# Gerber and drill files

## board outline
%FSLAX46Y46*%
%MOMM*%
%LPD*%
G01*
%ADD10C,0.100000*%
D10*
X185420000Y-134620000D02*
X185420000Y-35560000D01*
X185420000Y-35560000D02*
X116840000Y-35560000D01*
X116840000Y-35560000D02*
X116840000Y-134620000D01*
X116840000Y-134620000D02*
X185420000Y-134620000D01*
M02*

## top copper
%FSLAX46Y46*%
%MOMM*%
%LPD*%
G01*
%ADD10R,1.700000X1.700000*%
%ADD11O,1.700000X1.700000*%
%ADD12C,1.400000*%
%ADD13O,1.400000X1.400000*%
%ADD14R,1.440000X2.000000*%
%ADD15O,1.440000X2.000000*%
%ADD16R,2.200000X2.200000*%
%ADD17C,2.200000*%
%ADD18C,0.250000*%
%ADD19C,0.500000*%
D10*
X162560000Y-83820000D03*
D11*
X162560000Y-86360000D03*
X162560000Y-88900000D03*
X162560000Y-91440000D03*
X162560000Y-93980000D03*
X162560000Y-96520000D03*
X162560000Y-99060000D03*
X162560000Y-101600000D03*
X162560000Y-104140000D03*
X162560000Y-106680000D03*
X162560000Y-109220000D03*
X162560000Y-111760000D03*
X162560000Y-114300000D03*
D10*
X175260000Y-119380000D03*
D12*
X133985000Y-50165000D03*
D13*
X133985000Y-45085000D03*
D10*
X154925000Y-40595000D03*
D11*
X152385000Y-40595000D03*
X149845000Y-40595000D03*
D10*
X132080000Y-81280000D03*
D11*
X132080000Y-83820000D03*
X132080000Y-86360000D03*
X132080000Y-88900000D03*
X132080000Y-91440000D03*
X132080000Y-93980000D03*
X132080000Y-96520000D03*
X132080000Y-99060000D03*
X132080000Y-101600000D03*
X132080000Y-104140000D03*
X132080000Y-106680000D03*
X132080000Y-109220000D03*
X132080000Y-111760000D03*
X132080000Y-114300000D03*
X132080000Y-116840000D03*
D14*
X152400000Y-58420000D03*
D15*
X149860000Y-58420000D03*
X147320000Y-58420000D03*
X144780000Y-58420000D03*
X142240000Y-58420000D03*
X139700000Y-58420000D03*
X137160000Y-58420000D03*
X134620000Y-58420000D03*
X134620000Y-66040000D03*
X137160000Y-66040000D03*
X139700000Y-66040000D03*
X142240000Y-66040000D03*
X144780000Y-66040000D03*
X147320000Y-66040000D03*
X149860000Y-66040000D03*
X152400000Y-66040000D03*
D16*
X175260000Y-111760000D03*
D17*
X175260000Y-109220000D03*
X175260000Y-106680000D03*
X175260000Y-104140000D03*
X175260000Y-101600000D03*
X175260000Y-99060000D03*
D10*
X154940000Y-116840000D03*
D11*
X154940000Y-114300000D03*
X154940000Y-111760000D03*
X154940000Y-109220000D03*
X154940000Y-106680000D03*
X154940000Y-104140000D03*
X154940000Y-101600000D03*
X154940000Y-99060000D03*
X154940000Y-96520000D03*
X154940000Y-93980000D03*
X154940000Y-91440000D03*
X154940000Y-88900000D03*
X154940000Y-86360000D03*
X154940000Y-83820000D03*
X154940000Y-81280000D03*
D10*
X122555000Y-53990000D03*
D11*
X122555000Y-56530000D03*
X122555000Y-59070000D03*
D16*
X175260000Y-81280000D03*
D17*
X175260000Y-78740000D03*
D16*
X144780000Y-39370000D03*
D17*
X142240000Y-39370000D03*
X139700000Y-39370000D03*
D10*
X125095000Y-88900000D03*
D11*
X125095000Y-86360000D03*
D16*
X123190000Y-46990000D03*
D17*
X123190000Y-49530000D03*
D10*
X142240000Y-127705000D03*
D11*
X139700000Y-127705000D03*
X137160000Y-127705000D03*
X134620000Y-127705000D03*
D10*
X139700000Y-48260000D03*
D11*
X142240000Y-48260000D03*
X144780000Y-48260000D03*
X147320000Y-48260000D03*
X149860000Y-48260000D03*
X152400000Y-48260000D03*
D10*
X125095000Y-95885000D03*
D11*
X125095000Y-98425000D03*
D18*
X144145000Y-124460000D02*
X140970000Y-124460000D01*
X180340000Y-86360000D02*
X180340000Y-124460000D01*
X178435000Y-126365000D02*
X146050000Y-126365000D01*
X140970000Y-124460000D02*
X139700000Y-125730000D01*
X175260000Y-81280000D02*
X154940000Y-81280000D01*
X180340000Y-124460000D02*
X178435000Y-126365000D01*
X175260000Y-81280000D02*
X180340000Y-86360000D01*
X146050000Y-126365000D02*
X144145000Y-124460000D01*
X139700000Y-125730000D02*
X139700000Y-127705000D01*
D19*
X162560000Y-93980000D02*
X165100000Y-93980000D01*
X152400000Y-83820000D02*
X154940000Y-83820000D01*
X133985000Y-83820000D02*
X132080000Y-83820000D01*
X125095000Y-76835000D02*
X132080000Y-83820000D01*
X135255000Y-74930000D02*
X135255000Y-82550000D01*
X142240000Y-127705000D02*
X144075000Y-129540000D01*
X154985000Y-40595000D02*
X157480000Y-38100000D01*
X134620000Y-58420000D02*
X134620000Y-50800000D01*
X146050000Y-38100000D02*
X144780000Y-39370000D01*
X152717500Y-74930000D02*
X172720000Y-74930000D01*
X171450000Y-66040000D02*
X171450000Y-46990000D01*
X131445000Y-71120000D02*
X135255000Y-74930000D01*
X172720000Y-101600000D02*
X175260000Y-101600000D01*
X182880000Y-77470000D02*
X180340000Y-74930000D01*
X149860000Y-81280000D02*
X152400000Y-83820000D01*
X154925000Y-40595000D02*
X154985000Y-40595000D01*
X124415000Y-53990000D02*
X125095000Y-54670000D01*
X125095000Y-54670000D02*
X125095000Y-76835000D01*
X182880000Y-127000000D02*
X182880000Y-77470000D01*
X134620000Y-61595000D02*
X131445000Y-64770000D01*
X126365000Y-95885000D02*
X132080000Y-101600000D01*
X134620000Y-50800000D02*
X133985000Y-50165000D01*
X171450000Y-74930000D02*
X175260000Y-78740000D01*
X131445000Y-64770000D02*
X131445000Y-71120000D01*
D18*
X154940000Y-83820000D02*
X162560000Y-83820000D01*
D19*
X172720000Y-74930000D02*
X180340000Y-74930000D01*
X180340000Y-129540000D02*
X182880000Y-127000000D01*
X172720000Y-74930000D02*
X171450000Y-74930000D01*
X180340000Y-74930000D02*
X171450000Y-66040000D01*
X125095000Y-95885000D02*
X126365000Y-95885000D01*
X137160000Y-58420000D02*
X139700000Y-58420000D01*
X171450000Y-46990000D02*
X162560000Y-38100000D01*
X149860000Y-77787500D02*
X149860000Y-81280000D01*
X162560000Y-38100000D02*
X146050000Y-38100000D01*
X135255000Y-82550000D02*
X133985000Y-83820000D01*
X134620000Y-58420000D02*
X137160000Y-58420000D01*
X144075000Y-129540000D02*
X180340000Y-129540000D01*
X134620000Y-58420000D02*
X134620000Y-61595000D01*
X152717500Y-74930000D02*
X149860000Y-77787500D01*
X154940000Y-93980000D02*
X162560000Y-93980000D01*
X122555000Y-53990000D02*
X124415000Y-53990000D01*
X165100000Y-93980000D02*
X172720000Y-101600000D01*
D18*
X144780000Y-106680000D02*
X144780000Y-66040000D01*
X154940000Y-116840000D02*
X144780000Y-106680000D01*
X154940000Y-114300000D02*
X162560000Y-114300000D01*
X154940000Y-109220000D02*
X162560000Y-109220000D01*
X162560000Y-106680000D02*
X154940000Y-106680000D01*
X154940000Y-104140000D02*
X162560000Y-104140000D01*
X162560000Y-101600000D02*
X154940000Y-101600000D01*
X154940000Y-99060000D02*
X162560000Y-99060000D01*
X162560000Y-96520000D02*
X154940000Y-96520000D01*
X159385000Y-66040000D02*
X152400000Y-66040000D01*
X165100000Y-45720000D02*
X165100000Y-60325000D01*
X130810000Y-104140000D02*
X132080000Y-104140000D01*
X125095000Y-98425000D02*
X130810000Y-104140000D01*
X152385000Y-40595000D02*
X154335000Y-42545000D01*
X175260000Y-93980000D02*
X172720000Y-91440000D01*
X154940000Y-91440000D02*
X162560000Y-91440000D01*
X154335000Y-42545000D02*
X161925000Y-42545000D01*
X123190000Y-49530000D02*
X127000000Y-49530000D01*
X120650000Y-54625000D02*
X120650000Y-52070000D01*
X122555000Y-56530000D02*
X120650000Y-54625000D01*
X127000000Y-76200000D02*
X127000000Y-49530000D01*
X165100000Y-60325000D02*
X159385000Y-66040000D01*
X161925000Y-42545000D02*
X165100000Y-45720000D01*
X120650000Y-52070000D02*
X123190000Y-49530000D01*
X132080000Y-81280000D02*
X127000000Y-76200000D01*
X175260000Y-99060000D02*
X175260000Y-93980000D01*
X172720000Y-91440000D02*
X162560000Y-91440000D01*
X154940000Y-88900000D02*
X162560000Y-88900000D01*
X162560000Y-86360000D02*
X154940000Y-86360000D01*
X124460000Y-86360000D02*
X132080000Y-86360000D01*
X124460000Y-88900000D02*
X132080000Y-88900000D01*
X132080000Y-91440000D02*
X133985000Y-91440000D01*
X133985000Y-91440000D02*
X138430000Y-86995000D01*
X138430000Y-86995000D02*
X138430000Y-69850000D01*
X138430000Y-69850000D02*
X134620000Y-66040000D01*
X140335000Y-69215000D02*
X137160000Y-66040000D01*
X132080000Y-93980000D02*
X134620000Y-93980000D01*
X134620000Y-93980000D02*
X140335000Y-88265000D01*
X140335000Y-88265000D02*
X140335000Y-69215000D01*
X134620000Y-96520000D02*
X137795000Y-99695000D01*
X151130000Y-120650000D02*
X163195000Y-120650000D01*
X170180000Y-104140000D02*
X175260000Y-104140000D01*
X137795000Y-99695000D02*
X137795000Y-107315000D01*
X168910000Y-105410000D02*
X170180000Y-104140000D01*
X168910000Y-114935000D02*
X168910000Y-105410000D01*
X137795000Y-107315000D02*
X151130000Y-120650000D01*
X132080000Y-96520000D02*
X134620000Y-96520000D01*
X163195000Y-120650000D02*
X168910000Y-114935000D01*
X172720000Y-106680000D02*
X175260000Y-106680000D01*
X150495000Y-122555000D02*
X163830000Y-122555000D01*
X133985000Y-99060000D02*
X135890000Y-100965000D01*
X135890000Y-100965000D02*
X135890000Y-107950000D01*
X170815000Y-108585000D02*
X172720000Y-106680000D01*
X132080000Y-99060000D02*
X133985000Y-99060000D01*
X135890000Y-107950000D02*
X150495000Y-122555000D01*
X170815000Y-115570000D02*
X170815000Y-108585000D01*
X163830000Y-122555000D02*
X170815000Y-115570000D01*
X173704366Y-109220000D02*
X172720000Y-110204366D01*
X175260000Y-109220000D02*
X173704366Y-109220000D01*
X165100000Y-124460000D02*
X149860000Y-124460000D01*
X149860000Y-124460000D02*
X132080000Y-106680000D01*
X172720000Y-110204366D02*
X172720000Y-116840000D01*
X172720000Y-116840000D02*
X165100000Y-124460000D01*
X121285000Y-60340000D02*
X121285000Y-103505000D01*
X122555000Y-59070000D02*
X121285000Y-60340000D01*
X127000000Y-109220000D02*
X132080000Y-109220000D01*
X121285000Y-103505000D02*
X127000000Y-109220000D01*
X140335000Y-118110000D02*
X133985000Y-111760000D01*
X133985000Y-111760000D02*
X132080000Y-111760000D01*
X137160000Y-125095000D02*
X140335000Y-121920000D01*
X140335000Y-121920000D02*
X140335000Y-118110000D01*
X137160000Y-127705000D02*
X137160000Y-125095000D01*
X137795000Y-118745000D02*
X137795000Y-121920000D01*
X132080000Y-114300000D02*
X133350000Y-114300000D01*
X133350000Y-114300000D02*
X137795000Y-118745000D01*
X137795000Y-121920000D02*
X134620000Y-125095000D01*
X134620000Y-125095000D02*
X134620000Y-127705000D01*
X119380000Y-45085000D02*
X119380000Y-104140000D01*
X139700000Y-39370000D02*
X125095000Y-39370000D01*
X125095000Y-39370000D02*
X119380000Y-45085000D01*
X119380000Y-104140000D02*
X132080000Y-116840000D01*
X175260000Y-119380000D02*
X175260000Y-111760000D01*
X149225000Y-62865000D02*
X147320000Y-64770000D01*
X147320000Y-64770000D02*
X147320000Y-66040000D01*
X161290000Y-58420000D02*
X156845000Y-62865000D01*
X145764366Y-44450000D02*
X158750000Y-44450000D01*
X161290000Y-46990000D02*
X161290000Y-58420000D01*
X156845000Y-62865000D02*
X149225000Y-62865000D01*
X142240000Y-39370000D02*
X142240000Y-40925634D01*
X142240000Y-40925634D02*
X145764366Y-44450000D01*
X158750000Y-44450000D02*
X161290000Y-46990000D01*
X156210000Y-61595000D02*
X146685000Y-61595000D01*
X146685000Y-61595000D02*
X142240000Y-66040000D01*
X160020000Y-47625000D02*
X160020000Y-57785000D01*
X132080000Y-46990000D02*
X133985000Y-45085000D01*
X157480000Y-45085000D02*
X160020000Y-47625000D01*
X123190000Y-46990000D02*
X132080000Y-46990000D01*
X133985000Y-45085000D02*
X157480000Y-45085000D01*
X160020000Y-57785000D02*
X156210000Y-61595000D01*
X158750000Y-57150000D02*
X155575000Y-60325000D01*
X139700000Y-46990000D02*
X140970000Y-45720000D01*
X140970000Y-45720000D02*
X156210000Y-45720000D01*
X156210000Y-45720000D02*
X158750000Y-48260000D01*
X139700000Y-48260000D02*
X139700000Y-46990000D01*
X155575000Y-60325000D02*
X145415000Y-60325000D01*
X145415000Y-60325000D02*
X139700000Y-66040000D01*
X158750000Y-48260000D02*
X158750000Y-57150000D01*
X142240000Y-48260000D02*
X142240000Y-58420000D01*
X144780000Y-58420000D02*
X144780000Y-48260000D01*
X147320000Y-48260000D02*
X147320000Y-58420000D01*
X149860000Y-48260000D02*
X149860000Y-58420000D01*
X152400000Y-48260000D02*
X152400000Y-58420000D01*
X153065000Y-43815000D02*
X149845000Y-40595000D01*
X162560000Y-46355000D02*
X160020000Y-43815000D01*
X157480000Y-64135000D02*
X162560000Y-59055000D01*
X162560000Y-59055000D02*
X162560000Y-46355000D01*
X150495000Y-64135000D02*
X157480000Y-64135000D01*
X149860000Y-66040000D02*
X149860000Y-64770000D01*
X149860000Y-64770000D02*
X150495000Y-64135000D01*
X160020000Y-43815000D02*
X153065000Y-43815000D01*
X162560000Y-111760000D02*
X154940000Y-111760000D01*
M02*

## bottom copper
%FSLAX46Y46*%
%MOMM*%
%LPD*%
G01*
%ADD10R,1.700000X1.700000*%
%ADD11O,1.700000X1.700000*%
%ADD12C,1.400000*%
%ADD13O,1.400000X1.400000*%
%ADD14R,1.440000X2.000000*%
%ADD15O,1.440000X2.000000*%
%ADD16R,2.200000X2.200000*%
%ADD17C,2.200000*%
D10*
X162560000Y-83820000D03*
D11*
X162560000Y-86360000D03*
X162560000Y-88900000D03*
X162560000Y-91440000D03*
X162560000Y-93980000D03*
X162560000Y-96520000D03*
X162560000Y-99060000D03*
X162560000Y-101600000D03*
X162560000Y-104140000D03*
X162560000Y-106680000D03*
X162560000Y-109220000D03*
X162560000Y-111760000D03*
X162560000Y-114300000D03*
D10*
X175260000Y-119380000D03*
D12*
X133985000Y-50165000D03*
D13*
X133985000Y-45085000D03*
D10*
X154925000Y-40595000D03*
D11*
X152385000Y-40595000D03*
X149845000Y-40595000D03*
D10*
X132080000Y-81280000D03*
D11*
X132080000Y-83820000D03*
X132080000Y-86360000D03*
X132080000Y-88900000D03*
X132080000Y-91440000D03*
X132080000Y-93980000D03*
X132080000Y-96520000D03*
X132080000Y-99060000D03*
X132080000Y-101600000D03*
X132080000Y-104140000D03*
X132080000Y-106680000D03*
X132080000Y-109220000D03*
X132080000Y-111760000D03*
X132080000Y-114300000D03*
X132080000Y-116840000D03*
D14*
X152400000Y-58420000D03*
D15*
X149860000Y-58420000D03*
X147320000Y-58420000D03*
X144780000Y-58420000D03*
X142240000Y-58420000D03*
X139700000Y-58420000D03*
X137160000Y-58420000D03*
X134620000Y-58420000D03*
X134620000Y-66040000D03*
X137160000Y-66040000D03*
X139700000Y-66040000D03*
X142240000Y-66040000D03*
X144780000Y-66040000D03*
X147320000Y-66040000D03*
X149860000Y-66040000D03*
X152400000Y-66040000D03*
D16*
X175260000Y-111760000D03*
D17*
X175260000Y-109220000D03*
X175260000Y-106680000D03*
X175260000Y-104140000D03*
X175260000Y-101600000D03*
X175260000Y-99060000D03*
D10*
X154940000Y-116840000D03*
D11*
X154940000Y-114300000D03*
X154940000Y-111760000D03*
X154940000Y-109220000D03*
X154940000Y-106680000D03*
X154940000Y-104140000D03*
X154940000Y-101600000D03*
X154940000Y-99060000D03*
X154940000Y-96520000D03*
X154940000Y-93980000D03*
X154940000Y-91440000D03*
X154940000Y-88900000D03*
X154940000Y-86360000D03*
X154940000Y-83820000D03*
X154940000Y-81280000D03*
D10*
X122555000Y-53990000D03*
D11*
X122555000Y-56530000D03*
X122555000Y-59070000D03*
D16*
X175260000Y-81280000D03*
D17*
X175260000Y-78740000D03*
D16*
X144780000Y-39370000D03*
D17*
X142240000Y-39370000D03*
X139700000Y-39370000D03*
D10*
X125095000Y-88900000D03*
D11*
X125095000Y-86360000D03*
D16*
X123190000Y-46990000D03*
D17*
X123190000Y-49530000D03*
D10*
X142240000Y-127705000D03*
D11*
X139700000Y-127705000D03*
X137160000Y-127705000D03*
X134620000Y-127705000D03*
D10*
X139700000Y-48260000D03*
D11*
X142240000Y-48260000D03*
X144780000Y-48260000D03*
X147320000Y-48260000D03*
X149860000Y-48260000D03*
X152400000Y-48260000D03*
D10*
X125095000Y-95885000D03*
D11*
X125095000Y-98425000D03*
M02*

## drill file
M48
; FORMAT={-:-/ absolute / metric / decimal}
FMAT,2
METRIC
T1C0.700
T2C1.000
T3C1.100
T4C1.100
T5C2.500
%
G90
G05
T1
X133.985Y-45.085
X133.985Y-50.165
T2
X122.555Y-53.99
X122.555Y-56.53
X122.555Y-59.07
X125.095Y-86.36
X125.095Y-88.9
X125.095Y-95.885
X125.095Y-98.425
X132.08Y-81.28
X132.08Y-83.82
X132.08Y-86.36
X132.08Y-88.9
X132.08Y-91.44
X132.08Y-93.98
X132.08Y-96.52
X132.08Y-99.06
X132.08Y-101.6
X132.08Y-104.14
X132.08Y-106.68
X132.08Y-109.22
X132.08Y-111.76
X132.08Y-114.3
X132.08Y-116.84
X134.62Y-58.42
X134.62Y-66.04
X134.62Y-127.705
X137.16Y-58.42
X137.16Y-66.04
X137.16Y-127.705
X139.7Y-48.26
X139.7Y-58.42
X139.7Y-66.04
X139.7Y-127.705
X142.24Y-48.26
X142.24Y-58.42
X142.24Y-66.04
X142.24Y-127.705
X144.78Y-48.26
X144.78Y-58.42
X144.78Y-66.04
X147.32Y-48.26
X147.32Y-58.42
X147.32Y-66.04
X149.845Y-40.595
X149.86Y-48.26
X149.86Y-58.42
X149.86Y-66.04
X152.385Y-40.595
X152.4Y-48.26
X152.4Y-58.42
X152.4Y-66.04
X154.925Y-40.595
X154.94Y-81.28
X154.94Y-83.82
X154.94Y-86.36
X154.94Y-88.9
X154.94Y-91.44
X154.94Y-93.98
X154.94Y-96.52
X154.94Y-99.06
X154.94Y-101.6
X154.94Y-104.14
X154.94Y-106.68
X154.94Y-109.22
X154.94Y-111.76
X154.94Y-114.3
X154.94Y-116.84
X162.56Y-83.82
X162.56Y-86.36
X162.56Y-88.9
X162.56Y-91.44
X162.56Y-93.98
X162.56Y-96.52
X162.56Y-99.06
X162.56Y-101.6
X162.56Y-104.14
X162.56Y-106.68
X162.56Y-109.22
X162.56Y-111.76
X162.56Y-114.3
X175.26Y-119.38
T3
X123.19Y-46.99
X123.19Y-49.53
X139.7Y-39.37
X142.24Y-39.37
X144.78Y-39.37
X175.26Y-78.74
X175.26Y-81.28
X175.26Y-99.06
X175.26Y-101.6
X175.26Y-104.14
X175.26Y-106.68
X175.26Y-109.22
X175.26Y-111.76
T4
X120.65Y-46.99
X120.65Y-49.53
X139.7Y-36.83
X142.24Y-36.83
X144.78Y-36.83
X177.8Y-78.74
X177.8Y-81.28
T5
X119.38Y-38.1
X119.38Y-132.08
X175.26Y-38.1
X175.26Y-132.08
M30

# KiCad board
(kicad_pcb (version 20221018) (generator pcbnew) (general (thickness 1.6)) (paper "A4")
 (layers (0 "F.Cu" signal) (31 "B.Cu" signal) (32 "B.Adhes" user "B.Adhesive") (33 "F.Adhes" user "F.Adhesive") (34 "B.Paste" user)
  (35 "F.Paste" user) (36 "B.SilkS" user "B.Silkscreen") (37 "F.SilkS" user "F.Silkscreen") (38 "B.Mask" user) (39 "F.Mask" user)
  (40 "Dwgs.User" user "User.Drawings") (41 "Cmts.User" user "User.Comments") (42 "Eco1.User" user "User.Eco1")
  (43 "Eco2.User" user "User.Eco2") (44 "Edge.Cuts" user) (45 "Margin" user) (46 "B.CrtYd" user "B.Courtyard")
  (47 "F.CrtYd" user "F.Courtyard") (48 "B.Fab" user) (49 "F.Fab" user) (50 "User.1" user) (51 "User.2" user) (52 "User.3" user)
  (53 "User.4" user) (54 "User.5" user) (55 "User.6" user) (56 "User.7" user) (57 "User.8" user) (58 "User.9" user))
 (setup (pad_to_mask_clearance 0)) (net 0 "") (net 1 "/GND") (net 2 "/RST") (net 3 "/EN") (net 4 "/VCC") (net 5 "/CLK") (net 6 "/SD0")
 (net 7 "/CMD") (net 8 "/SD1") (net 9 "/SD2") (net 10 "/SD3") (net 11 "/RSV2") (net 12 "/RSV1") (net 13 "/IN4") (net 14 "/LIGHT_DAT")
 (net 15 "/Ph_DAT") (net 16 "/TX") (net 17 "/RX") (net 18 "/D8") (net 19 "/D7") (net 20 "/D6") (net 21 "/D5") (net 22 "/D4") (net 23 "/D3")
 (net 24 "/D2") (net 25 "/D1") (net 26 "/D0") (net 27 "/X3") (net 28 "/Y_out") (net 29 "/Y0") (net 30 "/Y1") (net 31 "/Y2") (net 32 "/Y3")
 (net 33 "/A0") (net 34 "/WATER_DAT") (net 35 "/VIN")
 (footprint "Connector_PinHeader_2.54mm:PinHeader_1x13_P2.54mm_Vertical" (layer "F.Cu") (at 162.56 83.82)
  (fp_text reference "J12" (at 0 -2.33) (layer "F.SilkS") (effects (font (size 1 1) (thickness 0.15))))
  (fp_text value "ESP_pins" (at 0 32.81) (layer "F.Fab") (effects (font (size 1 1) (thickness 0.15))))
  (pad "1" thru_hole rect (at 0 0) (size 1.7 1.7) (drill 1) (layers "*.Cu" "*.Mask") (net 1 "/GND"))
  (pad "2" thru_hole oval (at 0 2.54) (size 1.7 1.7) (drill 1) (layers "*.Cu" "*.Mask") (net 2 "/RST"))
  (pad "3" thru_hole oval (at 0 5.08) (size 1.7 1.7) (drill 1) (layers "*.Cu" "*.Mask") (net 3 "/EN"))
  (pad "4" thru_hole oval (at 0 7.62) (size 1.7 1.7) (drill 1) (layers "*.Cu" "*.Mask") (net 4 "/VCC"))
  (pad "5" thru_hole oval (at 0 10.16) (size 1.7 1.7) (drill 1) (layers "*.Cu" "*.Mask") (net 1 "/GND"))
  (pad "6" thru_hole oval (at 0 12.7) (size 1.7 1.7) (drill 1) (layers "*.Cu" "*.Mask") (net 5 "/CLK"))
  (pad "7" thru_hole oval (at 0 15.24) (size 1.7 1.7) (drill 1) (layers "*.Cu" "*.Mask") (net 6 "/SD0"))
  (pad "8" thru_hole oval (at 0 17.78) (size 1.7 1.7) (drill 1) (layers "*.Cu" "*.Mask") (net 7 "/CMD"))
  (pad "9" thru_hole oval (at 0 20.32) (size 1.7 1.7) (drill 1) (layers "*.Cu" "*.Mask") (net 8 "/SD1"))
  (pad "10" thru_hole oval (at 0 22.86) (size 1.7 1.7) (drill 1) (layers "*.Cu" "*.Mask") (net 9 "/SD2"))
  (pad "11" thru_hole oval (at 0 25.4) (size 1.7 1.7) (drill 1) (layers "*.Cu" "*.Mask") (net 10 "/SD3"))
  (pad "12" thru_hole oval (at 0 27.94) (size 1.7 1.7) (drill 1) (layers "*.Cu" "*.Mask") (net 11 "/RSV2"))
  (pad "13" thru_hole oval (at 0 30.48) (size 1.7 1.7) (drill 1) (layers "*.Cu" "*.Mask") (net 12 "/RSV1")))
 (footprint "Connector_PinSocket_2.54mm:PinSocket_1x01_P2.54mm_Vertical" (layer "F.Cu") (at 175.26 119.38)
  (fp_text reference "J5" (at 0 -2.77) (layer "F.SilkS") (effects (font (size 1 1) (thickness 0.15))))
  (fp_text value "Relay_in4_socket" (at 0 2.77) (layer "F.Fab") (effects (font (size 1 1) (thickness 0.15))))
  (pad "1" thru_hole rect (at 0 0) (size 1.7 1.7) (drill 1) (layers "*.Cu" "*.Mask") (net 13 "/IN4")))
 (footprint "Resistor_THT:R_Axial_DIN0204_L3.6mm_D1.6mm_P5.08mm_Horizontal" (layer "F.Cu") (at 133.985 50.165 90)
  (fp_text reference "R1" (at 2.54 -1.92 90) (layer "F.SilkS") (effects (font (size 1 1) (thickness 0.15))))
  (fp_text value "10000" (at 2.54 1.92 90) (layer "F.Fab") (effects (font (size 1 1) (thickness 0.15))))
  (pad "1" thru_hole circle (at 0 0 90) (size 1.4 1.4) (drill 0.7) (layers "*.Cu" "*.Mask") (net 1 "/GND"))
  (pad "2" thru_hole oval (at 5.08 0 90) (size 1.4 1.4) (drill 0.7) (layers "*.Cu" "*.Mask") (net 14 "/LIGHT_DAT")))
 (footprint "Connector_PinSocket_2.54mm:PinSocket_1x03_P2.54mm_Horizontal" (layer "F.Cu") (at 154.925 40.595 -90)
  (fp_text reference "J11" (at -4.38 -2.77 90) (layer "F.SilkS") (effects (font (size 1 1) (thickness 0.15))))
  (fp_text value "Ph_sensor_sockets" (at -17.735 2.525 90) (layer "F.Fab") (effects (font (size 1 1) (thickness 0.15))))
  (pad "1" thru_hole rect (at 0 0 270) (size 1.7 1.7) (drill 1) (layers "*.Cu" "*.Mask") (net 1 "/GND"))
  (pad "2" thru_hole oval (at 0 2.54 270) (size 1.7 1.7) (drill 1) (layers "*.Cu" "*.Mask") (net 4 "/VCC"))
  (pad "3" thru_hole oval (at 0 5.08 270) (size 1.7 1.7) (drill 1) (layers "*.Cu" "*.Mask") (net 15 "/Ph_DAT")))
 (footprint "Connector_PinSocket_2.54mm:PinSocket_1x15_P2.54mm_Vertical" (layer "F.Cu") (at 132.08 81.28)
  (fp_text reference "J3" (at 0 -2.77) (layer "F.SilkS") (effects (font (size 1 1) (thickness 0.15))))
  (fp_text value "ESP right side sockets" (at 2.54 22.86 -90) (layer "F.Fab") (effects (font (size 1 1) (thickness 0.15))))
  (pad "1" thru_hole rect (at 0 0) (size 1.7 1.7) (drill 1) (layers "*.Cu" "*.Mask") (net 4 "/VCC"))
  (pad "2" thru_hole oval (at 0 2.54) (size 1.7 1.7) (drill 1) (layers "*.Cu" "*.Mask") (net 1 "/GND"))
  (pad "3" thru_hole oval (at 0 5.08) (size 1.7 1.7) (drill 1) (layers "*.Cu" "*.Mask") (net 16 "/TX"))
  (pad "4" thru_hole oval (at 0 7.62) (size 1.7 1.7) (drill 1) (layers "*.Cu" "*.Mask") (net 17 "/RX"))
  (pad "5" thru_hole oval (at 0 10.16) (size 1.7 1.7) (drill 1) (layers "*.Cu" "*.Mask") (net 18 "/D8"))
  (pad "6" thru_hole oval (at 0 12.7) (size 1.7 1.7) (drill 1) (layers "*.Cu" "*.Mask") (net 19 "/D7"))
  (pad "7" thru_hole oval (at 0 15.24) (size 1.7 1.7) (drill 1) (layers "*.Cu" "*.Mask") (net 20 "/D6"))
  (pad "8" thru_hole oval (at 0 17.78) (size 1.7 1.7) (drill 1) (layers "*.Cu" "*.Mask") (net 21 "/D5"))
  (pad "9" thru_hole oval (at 0 20.32) (size 1.7 1.7) (drill 1) (layers "*.Cu" "*.Mask") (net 1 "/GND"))
  (pad "10" thru_hole oval (at 0 22.86) (size 1.7 1.7) (drill 1) (layers "*.Cu" "*.Mask") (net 4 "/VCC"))
  (pad "11" thru_hole oval (at 0 25.4) (size 1.7 1.7) (drill 1) (layers "*.Cu" "*.Mask") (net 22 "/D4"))
  (pad "12" thru_hole oval (at 0 27.94) (size 1.7 1.7) (drill 1) (layers "*.Cu" "*.Mask") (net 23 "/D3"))
  (pad "13" thru_hole oval (at 0 30.48) (size 1.7 1.7) (drill 1) (layers "*.Cu" "*.Mask") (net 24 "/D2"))
  (pad "14" thru_hole oval (at 0 33.02) (size 1.7 1.7) (drill 1) (layers "*.Cu" "*.Mask") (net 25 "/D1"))
  (pad "15" thru_hole oval (at 0 35.56) (size 1.7 1.7) (drill 1) (layers "*.Cu" "*.Mask") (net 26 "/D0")))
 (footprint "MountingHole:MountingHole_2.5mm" (layer "F.Cu") (at 119.38 38.1)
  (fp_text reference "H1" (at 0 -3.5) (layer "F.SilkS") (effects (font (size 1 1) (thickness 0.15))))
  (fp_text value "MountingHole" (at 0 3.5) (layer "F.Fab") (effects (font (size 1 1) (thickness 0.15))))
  (pad "" np_thru_hole circle (at 0 0) (size 2.5 2.5) (drill 2.5) (layers "*.Cu" "*.Mask")))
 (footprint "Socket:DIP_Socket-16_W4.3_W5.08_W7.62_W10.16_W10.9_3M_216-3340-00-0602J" (layer "F.Cu") (at 152.4 58.42 -90)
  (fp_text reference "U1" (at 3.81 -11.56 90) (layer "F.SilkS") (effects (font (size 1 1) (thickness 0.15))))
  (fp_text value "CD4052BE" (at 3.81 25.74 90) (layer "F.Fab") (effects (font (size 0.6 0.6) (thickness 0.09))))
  (pad "1" thru_hole rect (at 0 0 270) (size 2 1.44) (drill 1) (layers "*.Cu" "*.Mask") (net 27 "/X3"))
  (pad "2" thru_hole oval (at 0 2.54 270) (size 2 1.44) (drill 1) (layers "*.Cu" "*.Mask") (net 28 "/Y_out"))
  (pad "3" thru_hole oval (at 0 5.08 270) (size 2 1.44) (drill 1) (layers "*.Cu" "*.Mask") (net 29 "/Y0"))
  (pad "4" thru_hole oval (at 0 7.62 270) (size 2 1.44) (drill 1) (layers "*.Cu" "*.Mask") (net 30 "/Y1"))
  (pad "5" thru_hole oval (at 0 10.16 270) (size 2 1.44) (drill 1) (layers "*.Cu" "*.Mask") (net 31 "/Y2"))
  (pad "6" thru_hole oval (at 0 12.7 270) (size 2 1.44) (drill 1) (layers "*.Cu" "*.Mask") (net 1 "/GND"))
  (pad "7" thru_hole oval (at 0 15.24 270) (size 2 1.44) (drill 1) (layers "*.Cu" "*.Mask") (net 1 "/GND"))
  (pad "8" thru_hole oval (at 0 17.78 270) (size 2 1.44) (drill 1) (layers "*.Cu" "*.Mask") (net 1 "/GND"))
  (pad "9" thru_hole oval (at 7.62 17.78 270) (size 2 1.44) (drill 1) (layers "*.Cu" "*.Mask") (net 18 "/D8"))
  (pad "10" thru_hole oval (at 7.62 15.24 270) (size 2 1.44) (drill 1) (layers "*.Cu" "*.Mask") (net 19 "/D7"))
  (pad "11" thru_hole oval (at 7.62 12.7 270) (size 2 1.44) (drill 1) (layers "*.Cu" "*.Mask") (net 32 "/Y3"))
  (pad "12" thru_hole oval (at 7.62 10.16 270) (size 2 1.44) (drill 1) (layers "*.Cu" "*.Mask") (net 14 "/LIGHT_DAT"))
  (pad "13" thru_hole oval (at 7.62 7.62 270) (size 2 1.44) (drill 1) (layers "*.Cu" "*.Mask") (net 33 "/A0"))
  (pad "14" thru_hole oval (at 7.62 5.08 270) (size 2 1.44) (drill 1) (layers "*.Cu" "*.Mask") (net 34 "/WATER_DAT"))
  (pad "15" thru_hole oval (at 7.62 2.54 270) (size 2 1.44) (drill 1) (layers "*.Cu" "*.Mask") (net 15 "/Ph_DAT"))
  (pad "16" thru_hole oval (at 7.62 0 270) (size 2 1.44) (drill 1) (layers "*.Cu" "*.Mask") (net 4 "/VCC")))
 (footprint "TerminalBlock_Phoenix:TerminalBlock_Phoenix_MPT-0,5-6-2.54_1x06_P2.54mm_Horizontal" (layer "F.Cu") (at 175.26 111.76 90)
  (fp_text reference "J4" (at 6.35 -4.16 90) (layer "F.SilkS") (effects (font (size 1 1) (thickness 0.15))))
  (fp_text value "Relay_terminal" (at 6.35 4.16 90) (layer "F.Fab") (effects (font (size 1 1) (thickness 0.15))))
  (pad "1" thru_hole rect (at 0 0 90) (size 2.2 2.2) (drill 1.1) (layers "*.Cu" "*.Mask") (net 13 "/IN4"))
  (pad "2" thru_hole circle (at 2.54 0 90) (size 2.2 2.2) (drill 1.1) (layers "*.Cu" "*.Mask") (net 22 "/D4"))
  (pad "3" thru_hole circle (at 5.08 0 90) (size 2.2 2.2) (drill 1.1) (layers "*.Cu" "*.Mask") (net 21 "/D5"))
  (pad "4" thru_hole circle (at 7.62 0 90) (size 2.2 2.2) (drill 1.1) (layers "*.Cu" "*.Mask") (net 20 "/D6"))
  (pad "5" thru_hole circle (at 10.16 0 90) (size 2.2 2.2) (drill 1.1) (layers "*.Cu" "*.Mask") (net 1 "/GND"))
  (pad "6" thru_hole circle (at 12.7 0 90) (size 2.2 2.2) (drill 1.1) (layers "*.Cu" "*.Mask") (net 4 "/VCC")))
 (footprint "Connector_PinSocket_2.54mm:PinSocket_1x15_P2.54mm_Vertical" (layer "F.Cu") (at 154.94 116.84 180)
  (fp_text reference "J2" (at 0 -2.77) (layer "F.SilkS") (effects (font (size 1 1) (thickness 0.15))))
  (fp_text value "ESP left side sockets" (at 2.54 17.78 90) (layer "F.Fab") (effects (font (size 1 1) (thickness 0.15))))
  (pad "1" thru_hole rect (at 0 0 180) (size 1.7 1.7) (drill 1) (layers "*.Cu" "*.Mask") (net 33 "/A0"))
  (pad "2" thru_hole oval (at 0 2.54 180) (size 1.7 1.7) (drill 1) (layers "*.Cu" "*.Mask") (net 12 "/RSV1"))
  (pad "3" thru_hole oval (at 0 5.08 180) (size 1.7 1.7) (drill 1) (layers "*.Cu" "*.Mask") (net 11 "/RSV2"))
  (pad "4" thru_hole oval (at 0 7.62 180) (size 1.7 1.7) (drill 1) (layers "*.Cu" "*.Mask") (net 10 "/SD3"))
  (pad "5" thru_hole oval (at 0 10.16 180) (size 1.7 1.7) (drill 1) (layers "*.Cu" "*.Mask") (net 9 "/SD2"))
  (pad "6" thru_hole oval (at 0 12.7 180) (size 1.7 1.7) (drill 1) (layers "*.Cu" "*.Mask") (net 8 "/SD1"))
  (pad "7" thru_hole oval (at 0 15.24 180) (size 1.7 1.7) (drill 1) (layers "*.Cu" "*.Mask") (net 7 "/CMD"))
  (pad "8" thru_hole oval (at 0 17.78 180) (size 1.7 1.7) (drill 1) (layers "*.Cu" "*.Mask") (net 6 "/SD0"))
  (pad "9" thru_hole oval (at 0 20.32 180) (size 1.7 1.7) (drill 1) (layers "*.Cu" "*.Mask") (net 5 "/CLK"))
  (pad "10" thru_hole oval (at 0 22.86 180) (size 1.7 1.7) (drill 1) (layers "*.Cu" "*.Mask") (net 1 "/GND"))
  (pad "11" thru_hole oval (at 0 25.4 180) (size 1.7 1.7) (drill 1) (layers "*.Cu" "*.Mask") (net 4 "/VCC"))
  (pad "12" thru_hole oval (at 0 27.94 180) (size 1.7 1.7) (drill 1) (layers "*.Cu" "*.Mask") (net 3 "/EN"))
  (pad "13" thru_hole oval (at 0 30.48 180) (size 1.7 1.7) (drill 1) (layers "*.Cu" "*.Mask") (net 2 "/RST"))
  (pad "14" thru_hole oval (at 0 33.02 180) (size 1.7 1.7) (drill 1) (layers "*.Cu" "*.Mask") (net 1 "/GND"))
  (pad "15" thru_hole oval (at 0 35.56 180) (size 1.7 1.7) (drill 1) (layers "*.Cu" "*.Mask") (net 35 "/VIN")))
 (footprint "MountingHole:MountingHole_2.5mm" (layer "F.Cu") (at 175.26 132.08)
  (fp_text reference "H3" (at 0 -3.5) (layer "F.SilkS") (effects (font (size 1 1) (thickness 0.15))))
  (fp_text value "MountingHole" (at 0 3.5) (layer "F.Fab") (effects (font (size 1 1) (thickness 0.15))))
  (pad "" np_thru_hole circle (at 0 0) (size 2.5 2.5) (drill 2.5) (layers "*.Cu" "*.Mask")))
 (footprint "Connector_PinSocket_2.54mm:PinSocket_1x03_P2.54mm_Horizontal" (layer "F.Cu") (at 122.555 53.99)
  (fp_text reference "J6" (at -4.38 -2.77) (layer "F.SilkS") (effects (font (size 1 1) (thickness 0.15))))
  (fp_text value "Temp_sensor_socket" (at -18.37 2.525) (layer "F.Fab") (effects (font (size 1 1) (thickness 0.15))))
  (pad "1" thru_hole rect (at 0 0) (size 1.7 1.7) (drill 1) (layers "*.Cu" "*.Mask") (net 1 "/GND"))
  (pad "2" thru_hole oval (at 0 2.54) (size 1.7 1.7) (drill 1) (layers "*.Cu" "*.Mask") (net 4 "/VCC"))
  (pad "3" thru_hole oval (at 0 5.08) (size 1.7 1.7) (drill 1) (layers "*.Cu" "*.Mask") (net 23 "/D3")))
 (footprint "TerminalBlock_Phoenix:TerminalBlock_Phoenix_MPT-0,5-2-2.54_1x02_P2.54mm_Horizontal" (layer "F.Cu") (at 175.26 81.28 90)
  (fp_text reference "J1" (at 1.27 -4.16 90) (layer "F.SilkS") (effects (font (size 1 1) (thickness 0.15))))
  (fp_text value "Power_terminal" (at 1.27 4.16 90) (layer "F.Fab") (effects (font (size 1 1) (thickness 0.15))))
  (pad "" np_thru_hole circle (at 0 2.54 90) (size 1.1 1.1) (drill 1.1) (layers "*.Cu" "*.Mask"))
  (pad "" np_thru_hole circle (at 2.54 2.54 90) (size 1.1 1.1) (drill 1.1) (layers "*.Cu" "*.Mask"))
  (pad "1" thru_hole rect (at 0 0 90) (size 2.2 2.2) (drill 1.1) (layers "*.Cu" "*.Mask") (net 35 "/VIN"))
  (pad "2" thru_hole circle (at 2.54 0 90) (size 2.2 2.2) (drill 1.1) (layers "*.Cu" "*.Mask") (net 1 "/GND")))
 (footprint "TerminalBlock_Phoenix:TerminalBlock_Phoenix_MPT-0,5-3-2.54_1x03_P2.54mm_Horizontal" (layer "F.Cu") (at 144.78 39.37 180)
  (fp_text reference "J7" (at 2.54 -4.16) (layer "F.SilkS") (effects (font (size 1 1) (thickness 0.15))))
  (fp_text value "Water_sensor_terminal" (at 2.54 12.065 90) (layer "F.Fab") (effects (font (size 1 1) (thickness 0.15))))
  (pad "" np_thru_hole circle (at 0 2.54 180) (size 1.1 1.1) (drill 1.1) (layers "*.Cu" "*.Mask"))
  (pad "" np_thru_hole circle (at 2.54 2.54 180) (size 1.1 1.1) (drill 1.1) (layers "*.Cu" "*.Mask"))
  (pad "" np_thru_hole circle (at 5.08 2.54 180) (size 1.1 1.1) (drill 1.1) (layers "*.Cu" "*.Mask"))
  (pad "1" thru_hole rect (at 0 0 180) (size 2.2 2.2) (drill 1.1) (layers "*.Cu" "*.Mask") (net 1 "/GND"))
  (pad "2" thru_hole circle (at 2.54 0 180) (size 2.2 2.2) (drill 1.1) (layers "*.Cu" "*.Mask") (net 34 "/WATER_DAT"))
  (pad "3" thru_hole circle (at 5.08 0 180) (size 2.2 2.2) (drill 1.1) (layers "*.Cu" "*.Mask") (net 26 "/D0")))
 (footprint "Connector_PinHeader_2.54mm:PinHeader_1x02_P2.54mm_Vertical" (layer "F.Cu") (at 125.095 88.9 180)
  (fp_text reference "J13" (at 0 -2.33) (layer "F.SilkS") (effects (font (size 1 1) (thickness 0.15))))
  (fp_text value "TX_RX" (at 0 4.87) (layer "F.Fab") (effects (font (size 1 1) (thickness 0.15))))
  (pad "1" thru_hole rect (at 0 0 180) (size 1.7 1.7) (drill 1) (layers "*.Cu" "*.Mask") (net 17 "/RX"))
  (pad "2" thru_hole oval (at 0 2.54 180) (size 1.7 1.7) (drill 1) (layers "*.Cu" "*.Mask") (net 16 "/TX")))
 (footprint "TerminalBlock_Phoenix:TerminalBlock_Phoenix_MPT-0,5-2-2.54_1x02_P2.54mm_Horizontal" (layer "F.Cu") (at 123.19 46.99 -90)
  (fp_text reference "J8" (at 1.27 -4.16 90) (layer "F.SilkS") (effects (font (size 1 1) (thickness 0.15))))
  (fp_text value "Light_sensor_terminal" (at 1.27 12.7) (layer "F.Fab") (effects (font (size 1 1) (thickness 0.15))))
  (pad "" np_thru_hole circle (at 0 2.54 270) (size 1.1 1.1) (drill 1.1) (layers "*.Cu" "*.Mask"))
  (pad "" np_thru_hole circle (at 2.54 2.54 270) (size 1.1 1.1) (drill 1.1) (layers "*.Cu" "*.Mask"))
  (pad "1" thru_hole rect (at 0 0 270) (size 2.2 2.2) (drill 1.1) (layers "*.Cu" "*.Mask") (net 14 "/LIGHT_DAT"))
  (pad "2" thru_hole circle (at 2.54 0 270) (size 2.2 2.2) (drill 1.1) (layers "*.Cu" "*.Mask") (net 4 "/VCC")))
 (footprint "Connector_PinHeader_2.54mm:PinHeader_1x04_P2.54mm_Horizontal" (layer "F.Cu") (at 142.24 127.705 -90)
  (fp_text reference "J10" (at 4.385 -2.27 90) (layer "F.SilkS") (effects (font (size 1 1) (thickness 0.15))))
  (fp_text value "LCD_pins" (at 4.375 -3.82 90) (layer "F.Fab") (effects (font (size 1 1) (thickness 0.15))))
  (pad "1" thru_hole rect (at 0 0 270) (size 1.7 1.7) (drill 1) (layers "*.Cu" "*.Mask") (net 1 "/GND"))
  (pad "2" thru_hole oval (at 0 2.54 270) (size 1.7 1.7) (drill 1) (layers "*.Cu" "*.Mask") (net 35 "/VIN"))
  (pad "3" thru_hole oval (at 0 5.08 270) (size 1.7 1.7) (drill 1) (layers "*.Cu" "*.Mask") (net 24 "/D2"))
  (pad "4" thru_hole oval (at 0 7.62 270) (size 1.7 1.7) (drill 1) (layers "*.Cu" "*.Mask") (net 25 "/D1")))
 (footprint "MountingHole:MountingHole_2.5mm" (layer "F.Cu") (at 119.38 132.08)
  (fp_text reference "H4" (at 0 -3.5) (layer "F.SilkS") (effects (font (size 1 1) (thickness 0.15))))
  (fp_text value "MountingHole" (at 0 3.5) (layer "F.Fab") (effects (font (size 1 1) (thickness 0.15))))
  (pad "" np_thru_hole circle (at 0 0) (size 2.5 2.5) (drill 2.5) (layers "*.Cu" "*.Mask")))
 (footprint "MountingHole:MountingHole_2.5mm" (layer "F.Cu") (at 175.26 38.1)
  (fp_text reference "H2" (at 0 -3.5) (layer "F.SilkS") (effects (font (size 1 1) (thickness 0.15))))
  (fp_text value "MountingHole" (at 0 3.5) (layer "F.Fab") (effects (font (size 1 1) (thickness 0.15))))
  (pad "" np_thru_hole circle (at 0 0) (size 2.5 2.5) (drill 2.5) (layers "*.Cu" "*.Mask")))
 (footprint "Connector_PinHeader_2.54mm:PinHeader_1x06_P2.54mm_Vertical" (layer "F.Cu") (at 139.7 48.26 90)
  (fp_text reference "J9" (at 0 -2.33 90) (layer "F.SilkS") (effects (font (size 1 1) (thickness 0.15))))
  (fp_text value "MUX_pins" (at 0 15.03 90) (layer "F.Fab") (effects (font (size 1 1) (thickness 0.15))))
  (pad "1" thru_hole rect (at 0 0 90) (size 1.7 1.7) (drill 1) (layers "*.Cu" "*.Mask") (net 32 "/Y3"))
  (pad "2" thru_hole oval (at 0 2.54 90) (size 1.7 1.7) (drill 1) (layers "*.Cu" "*.Mask") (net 31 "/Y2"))
  (pad "3" thru_hole oval (at 0 5.08 90) (size 1.7 1.7) (drill 1) (layers "*.Cu" "*.Mask") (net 30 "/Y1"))
  (pad "4" thru_hole oval (at 0 7.62 90) (size 1.7 1.7) (drill 1) (layers "*.Cu" "*.Mask") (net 29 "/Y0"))
  (pad "5" thru_hole oval (at 0 10.16 90) (size 1.7 1.7) (drill 1) (layers "*.Cu" "*.Mask") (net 28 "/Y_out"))
  (pad "6" thru_hole oval (at 0 12.7 90) (size 1.7 1.7) (drill 1) (layers "*.Cu" "*.Mask") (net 27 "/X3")))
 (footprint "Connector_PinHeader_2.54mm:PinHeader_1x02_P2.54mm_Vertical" (layer "F.Cu") (at 125.095 95.885)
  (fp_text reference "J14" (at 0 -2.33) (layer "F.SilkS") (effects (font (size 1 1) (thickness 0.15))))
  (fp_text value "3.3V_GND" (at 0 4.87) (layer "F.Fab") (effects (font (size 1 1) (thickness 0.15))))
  (pad "1" thru_hole rect (at 0 0) (size 1.7 1.7) (drill 1) (layers "*.Cu" "*.Mask") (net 1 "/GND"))
  (pad "2" thru_hole oval (at 0 2.54) (size 1.7 1.7) (drill 1) (layers "*.Cu" "*.Mask") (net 4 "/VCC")))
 (gr_line (start 185.42 134.62) (end 185.42 35.56) (stroke (width 0.1) (type default)) (layer "Edge.Cuts"))
 (gr_line (start 185.42 35.56) (end 116.84 35.56) (stroke (width 0.1) (type default)) (layer "Edge.Cuts"))
 (gr_line (start 116.84 35.56) (end 116.84 134.62) (stroke (width 0.1) (type default)) (layer "Edge.Cuts"))
 (gr_line (start 116.84 134.62) (end 185.42 134.62) (stroke (width 0.1) (type default)) (layer "Edge.Cuts"))
 (segment (start 144.145 124.46) (end 140.97 124.46) (width 0.25) (layer "F.Cu") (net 35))
 (segment (start 180.34 86.36) (end 180.34 124.46) (width 0.25) (layer "F.Cu") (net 35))
 (segment (start 178.435 126.365) (end 146.05 126.365) (width 0.25) (layer "F.Cu") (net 35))
 (segment (start 140.97 124.46) (end 139.7 125.73) (width 0.25) (layer "F.Cu") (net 35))
 (segment (start 175.26 81.28) (end 154.94 81.28) (width 0.25) (layer "F.Cu") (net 35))
 (segment (start 180.34 124.46) (end 178.435 126.365) (width 0.25) (layer "F.Cu") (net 35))
 (segment (start 175.26 81.28) (end 180.34 86.36) (width 0.25) (layer "F.Cu") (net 35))
 (segment (start 146.05 126.365) (end 144.145 124.46) (width 0.25) (layer "F.Cu") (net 35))
 (segment (start 139.7 125.73) (end 139.7 127.705) (width 0.25) (layer "F.Cu") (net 35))
 (segment (start 162.56 93.98) (end 165.1 93.98) (width 0.5) (layer "F.Cu") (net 1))
 (segment (start 152.4 83.82) (end 154.94 83.82) (width 0.5) (layer "F.Cu") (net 1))
 (segment (start 133.985 83.82) (end 132.08 83.82) (width 0.5) (layer "F.Cu") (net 1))
 (segment (start 125.095 76.835) (end 132.08 83.82) (width 0.5) (layer "F.Cu") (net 1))
 (segment (start 135.255 74.93) (end 135.255 82.55) (width 0.5) (layer "F.Cu") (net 1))
 (segment (start 142.24 127.705) (end 144.075 129.54) (width 0.5) (layer "F.Cu") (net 1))
 (segment (start 154.985 40.595) (end 157.48 38.1) (width 0.5) (layer "F.Cu") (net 1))
 (segment (start 134.62 58.42) (end 134.62 50.8) (width 0.5) (layer "F.Cu") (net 1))
 (segment (start 146.05 38.1) (end 144.78 39.37) (width 0.5) (layer "F.Cu") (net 1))
 (segment (start 152.7175 74.93) (end 172.72 74.93) (width 0.5) (layer "F.Cu") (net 1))
 (segment (start 171.45 66.04) (end 171.45 46.99) (width 0.5) (layer "F.Cu") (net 1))
 (segment (start 131.445 71.12) (end 135.255 74.93) (width 0.5) (layer "F.Cu") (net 1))
 (segment (start 172.72 101.6) (end 175.26 101.6) (width 0.5) (layer "F.Cu") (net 1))
 (segment (start 182.88 77.47) (end 180.34 74.93) (width 0.5) (layer "F.Cu") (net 1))
 (segment (start 149.86 81.28) (end 152.4 83.82) (width 0.5) (layer "F.Cu") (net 1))
 (segment (start 154.925 40.595) (end 154.985 40.595) (width 0.5) (layer "F.Cu") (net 1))
 (segment (start 124.415 53.99) (end 125.095 54.67) (width 0.5) (layer "F.Cu") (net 1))
 (segment (start 125.095 54.67) (end 125.095 76.835) (width 0.5) (layer "F.Cu") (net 1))
 (segment (start 182.88 127) (end 182.88 77.47) (width 0.5) (layer "F.Cu") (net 1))
 (segment (start 134.62 61.595) (end 131.445 64.77) (width 0.5) (layer "F.Cu") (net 1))
 (segment (start 126.365 95.885) (end 132.08 101.6) (width 0.5) (layer "F.Cu") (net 1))
 (segment (start 134.62 50.8) (end 133.985 50.165) (width 0.5) (layer "F.Cu") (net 1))
 (segment (start 171.45 74.93) (end 175.26 78.74) (width 0.5) (layer "F.Cu") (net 1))
 (segment (start 131.445 64.77) (end 131.445 71.12) (width 0.5) (layer "F.Cu") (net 1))
 (segment (start 154.94 83.82) (end 162.56 83.82) (width 0.25) (layer "F.Cu") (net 1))
 (segment (start 172.72 74.93) (end 180.34 74.93) (width 0.5) (layer "F.Cu") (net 1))
 (segment (start 180.34 129.54) (end 182.88 127) (width 0.5) (layer "F.Cu") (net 1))
 (segment (start 172.72 74.93) (end 171.45 74.93) (width 0.5) (layer "F.Cu") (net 1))
 (segment (start 180.34 74.93) (end 171.45 66.04) (width 0.5) (layer "F.Cu") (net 1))
 (segment (start 125.095 95.885) (end 126.365 95.885) (width 0.5) (layer "F.Cu") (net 1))
 (segment (start 137.16 58.42) (end 139.7 58.42) (width 0.5) (layer "F.Cu") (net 1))
 (segment (start 171.45 46.99) (end 162.56 38.1) (width 0.5) (layer "F.Cu") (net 1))
 (segment (start 149.86 77.7875) (end 149.86 81.28) (width 0.5) (layer "F.Cu") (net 1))
 (segment (start 162.56 38.1) (end 146.05 38.1) (width 0.5) (layer "F.Cu") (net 1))
 (segment (start 135.255 82.55) (end 133.985 83.82) (width 0.5) (layer "F.Cu") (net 1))
 (segment (start 134.62 58.42) (end 137.16 58.42) (width 0.5) (layer "F.Cu") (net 1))
 (segment (start 144.075 129.54) (end 180.34 129.54) (width 0.5) (layer "F.Cu") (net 1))
 (segment (start 134.62 58.42) (end 134.62 61.595) (width 0.5) (layer "F.Cu") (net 1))
 (segment (start 152.7175 74.93) (end 149.86 77.7875) (width 0.5) (layer "F.Cu") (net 1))
 (segment (start 154.94 93.98) (end 162.56 93.98) (width 0.5) (layer "F.Cu") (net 1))
 (segment (start 122.555 53.99) (end 124.415 53.99) (width 0.5) (layer "F.Cu") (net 1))
 (segment (start 165.1 93.98) (end 172.72 101.6) (width 0.5) (layer "F.Cu") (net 1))
 (segment (start 144.78 106.68) (end 144.78 66.04) (width 0.25) (layer "F.Cu") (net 33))
 (segment (start 154.94 116.84) (end 144.78 106.68) (width 0.25) (layer "F.Cu") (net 33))
 (segment (start 154.94 114.3) (end 162.56 114.3) (width 0.25) (layer "F.Cu") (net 12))
 (segment (start 154.94 109.22) (end 162.56 109.22) (width 0.25) (layer "F.Cu") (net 10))
 (segment (start 162.56 106.68) (end 154.94 106.68) (width 0.25) (layer "F.Cu") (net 9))
 (segment (start 154.94 104.14) (end 162.56 104.14) (width 0.25) (layer "F.Cu") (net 8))
 (segment (start 162.56 101.6) (end 154.94 101.6) (width 0.25) (layer "F.Cu") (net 7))
 (segment (start 154.94 99.06) (end 162.56 99.06) (width 0.25) (layer "F.Cu") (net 6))
 (segment (start 162.56 96.52) (end 154.94 96.52) (width 0.25) (layer "F.Cu") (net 5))
 (segment (start 159.385 66.04) (end 152.4 66.04) (width 0.25) (layer "F.Cu") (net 4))
 (segment (start 165.1 45.72) (end 165.1 60.325) (width 0.25) (layer "F.Cu") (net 4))
 (segment (start 130.81 104.14) (end 132.08 104.14) (width 0.25) (layer "F.Cu") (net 4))
 (segment (start 125.095 98.425) (end 130.81 104.14) (width 0.25) (layer "F.Cu") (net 4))
 (segment (start 152.385 40.595) (end 154.335 42.545) (width 0.25) (layer "F.Cu") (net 4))
 (segment (start 175.26 93.98) (end 172.72 91.44) (width 0.25) (layer "F.Cu") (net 4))
 (segment (start 154.94 91.44) (end 162.56 91.44) (width 0.25) (layer "F.Cu") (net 4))
 (segment (start 154.335 42.545) (end 161.925 42.545) (width 0.25) (layer "F.Cu") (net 4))
 (segment (start 123.19 49.53) (end 127 49.53) (width 0.25) (layer "F.Cu") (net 4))
 (segment (start 120.65 54.625) (end 120.65 52.07) (width 0.25) (layer "F.Cu") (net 4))
 (segment (start 122.555 56.53) (end 120.65 54.625) (width 0.25) (layer "F.Cu") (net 4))
 (segment (start 127 76.2) (end 127 49.53) (width 0.25) (layer "F.Cu") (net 4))
 (segment (start 165.1 60.325) (end 159.385 66.04) (width 0.25) (layer "F.Cu") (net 4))
 (segment (start 161.925 42.545) (end 165.1 45.72) (width 0.25) (layer "F.Cu") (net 4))
 (segment (start 120.65 52.07) (end 123.19 49.53) (width 0.25) (layer "F.Cu") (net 4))
 (segment (start 132.08 81.28) (end 127 76.2) (width 0.25) (layer "F.Cu") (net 4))
 (segment (start 175.26 99.06) (end 175.26 93.98) (width 0.25) (layer "F.Cu") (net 4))
 (segment (start 172.72 91.44) (end 162.56 91.44) (width 0.25) (layer "F.Cu") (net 4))
 (segment (start 154.94 88.9) (end 162.56 88.9) (width 0.25) (layer "F.Cu") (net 3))
 (segment (start 162.56 86.36) (end 154.94 86.36) (width 0.25) (layer "F.Cu") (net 2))
 (segment (start 124.46 86.36) (end 132.08 86.36) (width 0.25) (layer "F.Cu") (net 16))
 (segment (start 124.46 88.9) (end 132.08 88.9) (width 0.25) (layer "F.Cu") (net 17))
 (segment (start 132.08 91.44) (end 133.985 91.44) (width 0.25) (layer "F.Cu") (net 18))
 (segment (start 133.985 91.44) (end 138.43 86.995) (width 0.25) (layer "F.Cu") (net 18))
 (segment (start 138.43 86.995) (end 138.43 69.85) (width 0.25) (layer "F.Cu") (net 18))
 (segment (start 138.43 69.85) (end 134.62 66.04) (width 0.25) (layer "F.Cu") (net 18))
 (segment (start 140.335 69.215) (end 137.16 66.04) (width 0.25) (layer "F.Cu") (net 19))
 (segment (start 132.08 93.98) (end 134.62 93.98) (width 0.25) (layer "F.Cu") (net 19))
 (segment (start 134.62 93.98) (end 140.335 88.265) (width 0.25) (layer "F.Cu") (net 19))
 (segment (start 140.335 88.265) (end 140.335 69.215) (width 0.25) (layer "F.Cu") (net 19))
 (segment (start 134.62 96.52) (end 137.795 99.695) (width 0.25) (layer "F.Cu") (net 20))
 (segment (start 151.13 120.65) (end 163.195 120.65) (width 0.25) (layer "F.Cu") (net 20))
 (segment (start 170.18 104.14) (end 175.26 104.14) (width 0.25) (layer "F.Cu") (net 20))
 (segment (start 137.795 99.695) (end 137.795 107.315) (width 0.25) (layer "F.Cu") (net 20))
 (segment (start 168.91 105.41) (end 170.18 104.14) (width 0.25) (layer "F.Cu") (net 20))
 (segment (start 168.91 114.935) (end 168.91 105.41) (width 0.25) (layer "F.Cu") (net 20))
 (segment (start 137.795 107.315) (end 151.13 120.65) (width 0.25) (layer "F.Cu") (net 20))
 (segment (start 132.08 96.52) (end 134.62 96.52) (width 0.25) (layer "F.Cu") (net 20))
 (segment (start 163.195 120.65) (end 168.91 114.935) (width 0.25) (layer "F.Cu") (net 20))
 (segment (start 172.72 106.68) (end 175.26 106.68) (width 0.25) (layer "F.Cu") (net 21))
 (segment (start 150.495 122.555) (end 163.83 122.555) (width 0.25) (layer "F.Cu") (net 21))
 (segment (start 133.985 99.06) (end 135.89 100.965) (width 0.25) (layer "F.Cu") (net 21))
 (segment (start 135.89 100.965) (end 135.89 107.95) (width 0.25) (layer "F.Cu") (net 21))
 (segment (start 170.815 108.585) (end 172.72 106.68) (width 0.25) (layer "F.Cu") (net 21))
 (segment (start 132.08 99.06) (end 133.985 99.06) (width 0.25) (layer "F.Cu") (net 21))
 (segment (start 135.89 107.95) (end 150.495 122.555) (width 0.25) (layer "F.Cu") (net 21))
 (segment (start 170.815 115.57) (end 170.815 108.585) (width 0.25) (layer "F.Cu") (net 21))
 (segment (start 163.83 122.555) (end 170.815 115.57) (width 0.25) (layer "F.Cu") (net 21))
 (segment (start 173.704366 109.22) (end 172.72 110.204366) (width 0.25) (layer "F.Cu") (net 22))
 (segment (start 175.26 109.22) (end 173.704366 109.22) (width 0.25) (layer "F.Cu") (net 22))
 (segment (start 165.1 124.46) (end 149.86 124.46) (width 0.25) (layer "F.Cu") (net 22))
 (segment (start 149.86 124.46) (end 132.08 106.68) (width 0.25) (layer "F.Cu") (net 22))
 (segment (start 172.72 110.204366) (end 172.72 116.84) (width 0.25) (layer "F.Cu") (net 22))
 (segment (start 172.72 116.84) (end 165.1 124.46) (width 0.25) (layer "F.Cu") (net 22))
 (segment (start 121.285 60.34) (end 121.285 103.505) (width 0.25) (layer "F.Cu") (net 23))
 (segment (start 122.555 59.07) (end 121.285 60.34) (width 0.25) (layer "F.Cu") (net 23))
 (segment (start 127 109.22) (end 132.08 109.22) (width 0.25) (layer "F.Cu") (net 23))
 (segment (start 121.285 103.505) (end 127 109.22) (width 0.25) (layer "F.Cu") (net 23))
 (segment (start 140.335 118.11) (end 133.985 111.76) (width 0.25) (layer "F.Cu") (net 24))
 (segment (start 133.985 111.76) (end 132.08 111.76) (width 0.25) (layer "F.Cu") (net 24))
 (segment (start 137.16 125.095) (end 140.335 121.92) (width 0.25) (layer "F.Cu") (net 24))
 (segment (start 140.335 121.92) (end 140.335 118.11) (width 0.25) (layer "F.Cu") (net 24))
 (segment (start 137.16 127.705) (end 137.16 125.095) (width 0.25) (layer "F.Cu") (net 24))
 (segment (start 137.795 118.745) (end 137.795 121.92) (width 0.25) (layer "F.Cu") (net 25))
 (segment (start 132.08 114.3) (end 133.35 114.3) (width 0.25) (layer "F.Cu") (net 25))
 (segment (start 133.35 114.3) (end 137.795 118.745) (width 0.25) (layer "F.Cu") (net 25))
 (segment (start 137.795 121.92) (end 134.62 125.095) (width 0.25) (layer "F.Cu") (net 25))
 (segment (start 134.62 125.095) (end 134.62 127.705) (width 0.25) (layer "F.Cu") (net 25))
 (segment (start 119.38 45.085) (end 119.38 104.14) (width 0.25) (layer "F.Cu") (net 26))
 (segment (start 139.7 39.37) (end 125.095 39.37) (width 0.25) (layer "F.Cu") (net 26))
 (segment (start 125.095 39.37) (end 119.38 45.085) (width 0.25) (layer "F.Cu") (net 26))
 (segment (start 119.38 104.14) (end 132.08 116.84) (width 0.25) (layer "F.Cu") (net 26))
 (segment (start 175.26 119.38) (end 175.26 111.76) (width 0.25) (layer "F.Cu") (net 13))
 (segment (start 149.225 62.865) (end 147.32 64.77) (width 0.25) (layer "F.Cu") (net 34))
 (segment (start 147.32 64.77) (end 147.32 66.04) (width 0.25) (layer "F.Cu") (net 34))
 (segment (start 161.29 58.42) (end 156.845 62.865) (width 0.25) (layer "F.Cu") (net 34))
 (segment (start 145.764366 44.45) (end 158.75 44.45) (width 0.25) (layer "F.Cu") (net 34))
 (segment (start 161.29 46.99) (end 161.29 58.42) (width 0.25) (layer "F.Cu") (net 34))
 (segment (start 156.845 62.865) (end 149.225 62.865) (width 0.25) (layer "F.Cu") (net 34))
 (segment (start 142.24 39.37) (end 142.24 40.925634) (width 0.25) (layer "F.Cu") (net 34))
 (segment (start 142.24 40.925634) (end 145.764366 44.45) (width 0.25) (layer "F.Cu") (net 34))
 (segment (start 158.75 44.45) (end 161.29 46.99) (width 0.25) (layer "F.Cu") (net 34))
 (segment (start 156.21 61.595) (end 146.685 61.595) (width 0.25) (layer "F.Cu") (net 14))
 (segment (start 146.685 61.595) (end 142.24 66.04) (width 0.25) (layer "F.Cu") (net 14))
 (segment (start 160.02 47.625) (end 160.02 57.785) (width 0.25) (layer "F.Cu") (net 14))
 (segment (start 132.08 46.99) (end 133.985 45.085) (width 0.25) (layer "F.Cu") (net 14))
 (segment (start 157.48 45.085) (end 160.02 47.625) (width 0.25) (layer "F.Cu") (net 14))
 (segment (start 123.19 46.99) (end 132.08 46.99) (width 0.25) (layer "F.Cu") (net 14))
 (segment (start 133.985 45.085) (end 157.48 45.085) (width 0.25) (layer "F.Cu") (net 14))
 (segment (start 160.02 57.785) (end 156.21 61.595) (width 0.25) (layer "F.Cu") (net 14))
 (segment (start 158.75 57.15) (end 155.575 60.325) (width 0.25) (layer "F.Cu") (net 32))
 (segment (start 139.7 46.99) (end 140.97 45.72) (width 0.25) (layer "F.Cu") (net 32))
 (segment (start 140.97 45.72) (end 156.21 45.72) (width 0.25) (layer "F.Cu") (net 32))
 (segment (start 156.21 45.72) (end 158.75 48.26) (width 0.25) (layer "F.Cu") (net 32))
 (segment (start 139.7 48.26) (end 139.7 46.99) (width 0.25) (layer "F.Cu") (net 32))
 (segment (start 155.575 60.325) (end 145.415 60.325) (width 0.25) (layer "F.Cu") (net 32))
 (segment (start 145.415 60.325) (end 139.7 66.04) (width 0.25) (layer "F.Cu") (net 32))
 (segment (start 158.75 48.26) (end 158.75 57.15) (width 0.25) (layer "F.Cu") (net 32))
 (segment (start 142.24 48.26) (end 142.24 58.42) (width 0.25) (layer "F.Cu") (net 31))
 (segment (start 144.78 58.42) (end 144.78 48.26) (width 0.25) (layer "F.Cu") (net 30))
 (segment (start 147.32 48.26) (end 147.32 58.42) (width 0.25) (layer "F.Cu") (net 29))
 (segment (start 149.86 48.26) (end 149.86 58.42) (width 0.25) (layer "F.Cu") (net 28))
 (segment (start 152.4 48.26) (end 152.4 58.42) (width 0.25) (layer "F.Cu") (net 27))
 (segment (start 153.065 43.815) (end 149.845 40.595) (width 0.25) (layer "F.Cu") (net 15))
 (segment (start 162.56 46.355) (end 160.02 43.815) (width 0.25) (layer "F.Cu") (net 15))
 (segment (start 157.48 64.135) (end 162.56 59.055) (width 0.25) (layer "F.Cu") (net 15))
 (segment (start 162.56 59.055) (end 162.56 46.355) (width 0.25) (layer "F.Cu") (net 15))
 (segment (start 150.495 64.135) (end 157.48 64.135) (width 0.25) (layer "F.Cu") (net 15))
 (segment (start 149.86 66.04) (end 149.86 64.77) (width 0.25) (layer "F.Cu") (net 15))
 (segment (start 149.86 64.77) (end 150.495 64.135) (width 0.25) (layer "F.Cu") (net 15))
 (segment (start 160.02 43.815) (end 153.065 43.815) (width 0.25) (layer "F.Cu") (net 15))
 (segment (start 162.56 111.76) (end 154.94 111.76) (width 0.25) (layer "F.Cu") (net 11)))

